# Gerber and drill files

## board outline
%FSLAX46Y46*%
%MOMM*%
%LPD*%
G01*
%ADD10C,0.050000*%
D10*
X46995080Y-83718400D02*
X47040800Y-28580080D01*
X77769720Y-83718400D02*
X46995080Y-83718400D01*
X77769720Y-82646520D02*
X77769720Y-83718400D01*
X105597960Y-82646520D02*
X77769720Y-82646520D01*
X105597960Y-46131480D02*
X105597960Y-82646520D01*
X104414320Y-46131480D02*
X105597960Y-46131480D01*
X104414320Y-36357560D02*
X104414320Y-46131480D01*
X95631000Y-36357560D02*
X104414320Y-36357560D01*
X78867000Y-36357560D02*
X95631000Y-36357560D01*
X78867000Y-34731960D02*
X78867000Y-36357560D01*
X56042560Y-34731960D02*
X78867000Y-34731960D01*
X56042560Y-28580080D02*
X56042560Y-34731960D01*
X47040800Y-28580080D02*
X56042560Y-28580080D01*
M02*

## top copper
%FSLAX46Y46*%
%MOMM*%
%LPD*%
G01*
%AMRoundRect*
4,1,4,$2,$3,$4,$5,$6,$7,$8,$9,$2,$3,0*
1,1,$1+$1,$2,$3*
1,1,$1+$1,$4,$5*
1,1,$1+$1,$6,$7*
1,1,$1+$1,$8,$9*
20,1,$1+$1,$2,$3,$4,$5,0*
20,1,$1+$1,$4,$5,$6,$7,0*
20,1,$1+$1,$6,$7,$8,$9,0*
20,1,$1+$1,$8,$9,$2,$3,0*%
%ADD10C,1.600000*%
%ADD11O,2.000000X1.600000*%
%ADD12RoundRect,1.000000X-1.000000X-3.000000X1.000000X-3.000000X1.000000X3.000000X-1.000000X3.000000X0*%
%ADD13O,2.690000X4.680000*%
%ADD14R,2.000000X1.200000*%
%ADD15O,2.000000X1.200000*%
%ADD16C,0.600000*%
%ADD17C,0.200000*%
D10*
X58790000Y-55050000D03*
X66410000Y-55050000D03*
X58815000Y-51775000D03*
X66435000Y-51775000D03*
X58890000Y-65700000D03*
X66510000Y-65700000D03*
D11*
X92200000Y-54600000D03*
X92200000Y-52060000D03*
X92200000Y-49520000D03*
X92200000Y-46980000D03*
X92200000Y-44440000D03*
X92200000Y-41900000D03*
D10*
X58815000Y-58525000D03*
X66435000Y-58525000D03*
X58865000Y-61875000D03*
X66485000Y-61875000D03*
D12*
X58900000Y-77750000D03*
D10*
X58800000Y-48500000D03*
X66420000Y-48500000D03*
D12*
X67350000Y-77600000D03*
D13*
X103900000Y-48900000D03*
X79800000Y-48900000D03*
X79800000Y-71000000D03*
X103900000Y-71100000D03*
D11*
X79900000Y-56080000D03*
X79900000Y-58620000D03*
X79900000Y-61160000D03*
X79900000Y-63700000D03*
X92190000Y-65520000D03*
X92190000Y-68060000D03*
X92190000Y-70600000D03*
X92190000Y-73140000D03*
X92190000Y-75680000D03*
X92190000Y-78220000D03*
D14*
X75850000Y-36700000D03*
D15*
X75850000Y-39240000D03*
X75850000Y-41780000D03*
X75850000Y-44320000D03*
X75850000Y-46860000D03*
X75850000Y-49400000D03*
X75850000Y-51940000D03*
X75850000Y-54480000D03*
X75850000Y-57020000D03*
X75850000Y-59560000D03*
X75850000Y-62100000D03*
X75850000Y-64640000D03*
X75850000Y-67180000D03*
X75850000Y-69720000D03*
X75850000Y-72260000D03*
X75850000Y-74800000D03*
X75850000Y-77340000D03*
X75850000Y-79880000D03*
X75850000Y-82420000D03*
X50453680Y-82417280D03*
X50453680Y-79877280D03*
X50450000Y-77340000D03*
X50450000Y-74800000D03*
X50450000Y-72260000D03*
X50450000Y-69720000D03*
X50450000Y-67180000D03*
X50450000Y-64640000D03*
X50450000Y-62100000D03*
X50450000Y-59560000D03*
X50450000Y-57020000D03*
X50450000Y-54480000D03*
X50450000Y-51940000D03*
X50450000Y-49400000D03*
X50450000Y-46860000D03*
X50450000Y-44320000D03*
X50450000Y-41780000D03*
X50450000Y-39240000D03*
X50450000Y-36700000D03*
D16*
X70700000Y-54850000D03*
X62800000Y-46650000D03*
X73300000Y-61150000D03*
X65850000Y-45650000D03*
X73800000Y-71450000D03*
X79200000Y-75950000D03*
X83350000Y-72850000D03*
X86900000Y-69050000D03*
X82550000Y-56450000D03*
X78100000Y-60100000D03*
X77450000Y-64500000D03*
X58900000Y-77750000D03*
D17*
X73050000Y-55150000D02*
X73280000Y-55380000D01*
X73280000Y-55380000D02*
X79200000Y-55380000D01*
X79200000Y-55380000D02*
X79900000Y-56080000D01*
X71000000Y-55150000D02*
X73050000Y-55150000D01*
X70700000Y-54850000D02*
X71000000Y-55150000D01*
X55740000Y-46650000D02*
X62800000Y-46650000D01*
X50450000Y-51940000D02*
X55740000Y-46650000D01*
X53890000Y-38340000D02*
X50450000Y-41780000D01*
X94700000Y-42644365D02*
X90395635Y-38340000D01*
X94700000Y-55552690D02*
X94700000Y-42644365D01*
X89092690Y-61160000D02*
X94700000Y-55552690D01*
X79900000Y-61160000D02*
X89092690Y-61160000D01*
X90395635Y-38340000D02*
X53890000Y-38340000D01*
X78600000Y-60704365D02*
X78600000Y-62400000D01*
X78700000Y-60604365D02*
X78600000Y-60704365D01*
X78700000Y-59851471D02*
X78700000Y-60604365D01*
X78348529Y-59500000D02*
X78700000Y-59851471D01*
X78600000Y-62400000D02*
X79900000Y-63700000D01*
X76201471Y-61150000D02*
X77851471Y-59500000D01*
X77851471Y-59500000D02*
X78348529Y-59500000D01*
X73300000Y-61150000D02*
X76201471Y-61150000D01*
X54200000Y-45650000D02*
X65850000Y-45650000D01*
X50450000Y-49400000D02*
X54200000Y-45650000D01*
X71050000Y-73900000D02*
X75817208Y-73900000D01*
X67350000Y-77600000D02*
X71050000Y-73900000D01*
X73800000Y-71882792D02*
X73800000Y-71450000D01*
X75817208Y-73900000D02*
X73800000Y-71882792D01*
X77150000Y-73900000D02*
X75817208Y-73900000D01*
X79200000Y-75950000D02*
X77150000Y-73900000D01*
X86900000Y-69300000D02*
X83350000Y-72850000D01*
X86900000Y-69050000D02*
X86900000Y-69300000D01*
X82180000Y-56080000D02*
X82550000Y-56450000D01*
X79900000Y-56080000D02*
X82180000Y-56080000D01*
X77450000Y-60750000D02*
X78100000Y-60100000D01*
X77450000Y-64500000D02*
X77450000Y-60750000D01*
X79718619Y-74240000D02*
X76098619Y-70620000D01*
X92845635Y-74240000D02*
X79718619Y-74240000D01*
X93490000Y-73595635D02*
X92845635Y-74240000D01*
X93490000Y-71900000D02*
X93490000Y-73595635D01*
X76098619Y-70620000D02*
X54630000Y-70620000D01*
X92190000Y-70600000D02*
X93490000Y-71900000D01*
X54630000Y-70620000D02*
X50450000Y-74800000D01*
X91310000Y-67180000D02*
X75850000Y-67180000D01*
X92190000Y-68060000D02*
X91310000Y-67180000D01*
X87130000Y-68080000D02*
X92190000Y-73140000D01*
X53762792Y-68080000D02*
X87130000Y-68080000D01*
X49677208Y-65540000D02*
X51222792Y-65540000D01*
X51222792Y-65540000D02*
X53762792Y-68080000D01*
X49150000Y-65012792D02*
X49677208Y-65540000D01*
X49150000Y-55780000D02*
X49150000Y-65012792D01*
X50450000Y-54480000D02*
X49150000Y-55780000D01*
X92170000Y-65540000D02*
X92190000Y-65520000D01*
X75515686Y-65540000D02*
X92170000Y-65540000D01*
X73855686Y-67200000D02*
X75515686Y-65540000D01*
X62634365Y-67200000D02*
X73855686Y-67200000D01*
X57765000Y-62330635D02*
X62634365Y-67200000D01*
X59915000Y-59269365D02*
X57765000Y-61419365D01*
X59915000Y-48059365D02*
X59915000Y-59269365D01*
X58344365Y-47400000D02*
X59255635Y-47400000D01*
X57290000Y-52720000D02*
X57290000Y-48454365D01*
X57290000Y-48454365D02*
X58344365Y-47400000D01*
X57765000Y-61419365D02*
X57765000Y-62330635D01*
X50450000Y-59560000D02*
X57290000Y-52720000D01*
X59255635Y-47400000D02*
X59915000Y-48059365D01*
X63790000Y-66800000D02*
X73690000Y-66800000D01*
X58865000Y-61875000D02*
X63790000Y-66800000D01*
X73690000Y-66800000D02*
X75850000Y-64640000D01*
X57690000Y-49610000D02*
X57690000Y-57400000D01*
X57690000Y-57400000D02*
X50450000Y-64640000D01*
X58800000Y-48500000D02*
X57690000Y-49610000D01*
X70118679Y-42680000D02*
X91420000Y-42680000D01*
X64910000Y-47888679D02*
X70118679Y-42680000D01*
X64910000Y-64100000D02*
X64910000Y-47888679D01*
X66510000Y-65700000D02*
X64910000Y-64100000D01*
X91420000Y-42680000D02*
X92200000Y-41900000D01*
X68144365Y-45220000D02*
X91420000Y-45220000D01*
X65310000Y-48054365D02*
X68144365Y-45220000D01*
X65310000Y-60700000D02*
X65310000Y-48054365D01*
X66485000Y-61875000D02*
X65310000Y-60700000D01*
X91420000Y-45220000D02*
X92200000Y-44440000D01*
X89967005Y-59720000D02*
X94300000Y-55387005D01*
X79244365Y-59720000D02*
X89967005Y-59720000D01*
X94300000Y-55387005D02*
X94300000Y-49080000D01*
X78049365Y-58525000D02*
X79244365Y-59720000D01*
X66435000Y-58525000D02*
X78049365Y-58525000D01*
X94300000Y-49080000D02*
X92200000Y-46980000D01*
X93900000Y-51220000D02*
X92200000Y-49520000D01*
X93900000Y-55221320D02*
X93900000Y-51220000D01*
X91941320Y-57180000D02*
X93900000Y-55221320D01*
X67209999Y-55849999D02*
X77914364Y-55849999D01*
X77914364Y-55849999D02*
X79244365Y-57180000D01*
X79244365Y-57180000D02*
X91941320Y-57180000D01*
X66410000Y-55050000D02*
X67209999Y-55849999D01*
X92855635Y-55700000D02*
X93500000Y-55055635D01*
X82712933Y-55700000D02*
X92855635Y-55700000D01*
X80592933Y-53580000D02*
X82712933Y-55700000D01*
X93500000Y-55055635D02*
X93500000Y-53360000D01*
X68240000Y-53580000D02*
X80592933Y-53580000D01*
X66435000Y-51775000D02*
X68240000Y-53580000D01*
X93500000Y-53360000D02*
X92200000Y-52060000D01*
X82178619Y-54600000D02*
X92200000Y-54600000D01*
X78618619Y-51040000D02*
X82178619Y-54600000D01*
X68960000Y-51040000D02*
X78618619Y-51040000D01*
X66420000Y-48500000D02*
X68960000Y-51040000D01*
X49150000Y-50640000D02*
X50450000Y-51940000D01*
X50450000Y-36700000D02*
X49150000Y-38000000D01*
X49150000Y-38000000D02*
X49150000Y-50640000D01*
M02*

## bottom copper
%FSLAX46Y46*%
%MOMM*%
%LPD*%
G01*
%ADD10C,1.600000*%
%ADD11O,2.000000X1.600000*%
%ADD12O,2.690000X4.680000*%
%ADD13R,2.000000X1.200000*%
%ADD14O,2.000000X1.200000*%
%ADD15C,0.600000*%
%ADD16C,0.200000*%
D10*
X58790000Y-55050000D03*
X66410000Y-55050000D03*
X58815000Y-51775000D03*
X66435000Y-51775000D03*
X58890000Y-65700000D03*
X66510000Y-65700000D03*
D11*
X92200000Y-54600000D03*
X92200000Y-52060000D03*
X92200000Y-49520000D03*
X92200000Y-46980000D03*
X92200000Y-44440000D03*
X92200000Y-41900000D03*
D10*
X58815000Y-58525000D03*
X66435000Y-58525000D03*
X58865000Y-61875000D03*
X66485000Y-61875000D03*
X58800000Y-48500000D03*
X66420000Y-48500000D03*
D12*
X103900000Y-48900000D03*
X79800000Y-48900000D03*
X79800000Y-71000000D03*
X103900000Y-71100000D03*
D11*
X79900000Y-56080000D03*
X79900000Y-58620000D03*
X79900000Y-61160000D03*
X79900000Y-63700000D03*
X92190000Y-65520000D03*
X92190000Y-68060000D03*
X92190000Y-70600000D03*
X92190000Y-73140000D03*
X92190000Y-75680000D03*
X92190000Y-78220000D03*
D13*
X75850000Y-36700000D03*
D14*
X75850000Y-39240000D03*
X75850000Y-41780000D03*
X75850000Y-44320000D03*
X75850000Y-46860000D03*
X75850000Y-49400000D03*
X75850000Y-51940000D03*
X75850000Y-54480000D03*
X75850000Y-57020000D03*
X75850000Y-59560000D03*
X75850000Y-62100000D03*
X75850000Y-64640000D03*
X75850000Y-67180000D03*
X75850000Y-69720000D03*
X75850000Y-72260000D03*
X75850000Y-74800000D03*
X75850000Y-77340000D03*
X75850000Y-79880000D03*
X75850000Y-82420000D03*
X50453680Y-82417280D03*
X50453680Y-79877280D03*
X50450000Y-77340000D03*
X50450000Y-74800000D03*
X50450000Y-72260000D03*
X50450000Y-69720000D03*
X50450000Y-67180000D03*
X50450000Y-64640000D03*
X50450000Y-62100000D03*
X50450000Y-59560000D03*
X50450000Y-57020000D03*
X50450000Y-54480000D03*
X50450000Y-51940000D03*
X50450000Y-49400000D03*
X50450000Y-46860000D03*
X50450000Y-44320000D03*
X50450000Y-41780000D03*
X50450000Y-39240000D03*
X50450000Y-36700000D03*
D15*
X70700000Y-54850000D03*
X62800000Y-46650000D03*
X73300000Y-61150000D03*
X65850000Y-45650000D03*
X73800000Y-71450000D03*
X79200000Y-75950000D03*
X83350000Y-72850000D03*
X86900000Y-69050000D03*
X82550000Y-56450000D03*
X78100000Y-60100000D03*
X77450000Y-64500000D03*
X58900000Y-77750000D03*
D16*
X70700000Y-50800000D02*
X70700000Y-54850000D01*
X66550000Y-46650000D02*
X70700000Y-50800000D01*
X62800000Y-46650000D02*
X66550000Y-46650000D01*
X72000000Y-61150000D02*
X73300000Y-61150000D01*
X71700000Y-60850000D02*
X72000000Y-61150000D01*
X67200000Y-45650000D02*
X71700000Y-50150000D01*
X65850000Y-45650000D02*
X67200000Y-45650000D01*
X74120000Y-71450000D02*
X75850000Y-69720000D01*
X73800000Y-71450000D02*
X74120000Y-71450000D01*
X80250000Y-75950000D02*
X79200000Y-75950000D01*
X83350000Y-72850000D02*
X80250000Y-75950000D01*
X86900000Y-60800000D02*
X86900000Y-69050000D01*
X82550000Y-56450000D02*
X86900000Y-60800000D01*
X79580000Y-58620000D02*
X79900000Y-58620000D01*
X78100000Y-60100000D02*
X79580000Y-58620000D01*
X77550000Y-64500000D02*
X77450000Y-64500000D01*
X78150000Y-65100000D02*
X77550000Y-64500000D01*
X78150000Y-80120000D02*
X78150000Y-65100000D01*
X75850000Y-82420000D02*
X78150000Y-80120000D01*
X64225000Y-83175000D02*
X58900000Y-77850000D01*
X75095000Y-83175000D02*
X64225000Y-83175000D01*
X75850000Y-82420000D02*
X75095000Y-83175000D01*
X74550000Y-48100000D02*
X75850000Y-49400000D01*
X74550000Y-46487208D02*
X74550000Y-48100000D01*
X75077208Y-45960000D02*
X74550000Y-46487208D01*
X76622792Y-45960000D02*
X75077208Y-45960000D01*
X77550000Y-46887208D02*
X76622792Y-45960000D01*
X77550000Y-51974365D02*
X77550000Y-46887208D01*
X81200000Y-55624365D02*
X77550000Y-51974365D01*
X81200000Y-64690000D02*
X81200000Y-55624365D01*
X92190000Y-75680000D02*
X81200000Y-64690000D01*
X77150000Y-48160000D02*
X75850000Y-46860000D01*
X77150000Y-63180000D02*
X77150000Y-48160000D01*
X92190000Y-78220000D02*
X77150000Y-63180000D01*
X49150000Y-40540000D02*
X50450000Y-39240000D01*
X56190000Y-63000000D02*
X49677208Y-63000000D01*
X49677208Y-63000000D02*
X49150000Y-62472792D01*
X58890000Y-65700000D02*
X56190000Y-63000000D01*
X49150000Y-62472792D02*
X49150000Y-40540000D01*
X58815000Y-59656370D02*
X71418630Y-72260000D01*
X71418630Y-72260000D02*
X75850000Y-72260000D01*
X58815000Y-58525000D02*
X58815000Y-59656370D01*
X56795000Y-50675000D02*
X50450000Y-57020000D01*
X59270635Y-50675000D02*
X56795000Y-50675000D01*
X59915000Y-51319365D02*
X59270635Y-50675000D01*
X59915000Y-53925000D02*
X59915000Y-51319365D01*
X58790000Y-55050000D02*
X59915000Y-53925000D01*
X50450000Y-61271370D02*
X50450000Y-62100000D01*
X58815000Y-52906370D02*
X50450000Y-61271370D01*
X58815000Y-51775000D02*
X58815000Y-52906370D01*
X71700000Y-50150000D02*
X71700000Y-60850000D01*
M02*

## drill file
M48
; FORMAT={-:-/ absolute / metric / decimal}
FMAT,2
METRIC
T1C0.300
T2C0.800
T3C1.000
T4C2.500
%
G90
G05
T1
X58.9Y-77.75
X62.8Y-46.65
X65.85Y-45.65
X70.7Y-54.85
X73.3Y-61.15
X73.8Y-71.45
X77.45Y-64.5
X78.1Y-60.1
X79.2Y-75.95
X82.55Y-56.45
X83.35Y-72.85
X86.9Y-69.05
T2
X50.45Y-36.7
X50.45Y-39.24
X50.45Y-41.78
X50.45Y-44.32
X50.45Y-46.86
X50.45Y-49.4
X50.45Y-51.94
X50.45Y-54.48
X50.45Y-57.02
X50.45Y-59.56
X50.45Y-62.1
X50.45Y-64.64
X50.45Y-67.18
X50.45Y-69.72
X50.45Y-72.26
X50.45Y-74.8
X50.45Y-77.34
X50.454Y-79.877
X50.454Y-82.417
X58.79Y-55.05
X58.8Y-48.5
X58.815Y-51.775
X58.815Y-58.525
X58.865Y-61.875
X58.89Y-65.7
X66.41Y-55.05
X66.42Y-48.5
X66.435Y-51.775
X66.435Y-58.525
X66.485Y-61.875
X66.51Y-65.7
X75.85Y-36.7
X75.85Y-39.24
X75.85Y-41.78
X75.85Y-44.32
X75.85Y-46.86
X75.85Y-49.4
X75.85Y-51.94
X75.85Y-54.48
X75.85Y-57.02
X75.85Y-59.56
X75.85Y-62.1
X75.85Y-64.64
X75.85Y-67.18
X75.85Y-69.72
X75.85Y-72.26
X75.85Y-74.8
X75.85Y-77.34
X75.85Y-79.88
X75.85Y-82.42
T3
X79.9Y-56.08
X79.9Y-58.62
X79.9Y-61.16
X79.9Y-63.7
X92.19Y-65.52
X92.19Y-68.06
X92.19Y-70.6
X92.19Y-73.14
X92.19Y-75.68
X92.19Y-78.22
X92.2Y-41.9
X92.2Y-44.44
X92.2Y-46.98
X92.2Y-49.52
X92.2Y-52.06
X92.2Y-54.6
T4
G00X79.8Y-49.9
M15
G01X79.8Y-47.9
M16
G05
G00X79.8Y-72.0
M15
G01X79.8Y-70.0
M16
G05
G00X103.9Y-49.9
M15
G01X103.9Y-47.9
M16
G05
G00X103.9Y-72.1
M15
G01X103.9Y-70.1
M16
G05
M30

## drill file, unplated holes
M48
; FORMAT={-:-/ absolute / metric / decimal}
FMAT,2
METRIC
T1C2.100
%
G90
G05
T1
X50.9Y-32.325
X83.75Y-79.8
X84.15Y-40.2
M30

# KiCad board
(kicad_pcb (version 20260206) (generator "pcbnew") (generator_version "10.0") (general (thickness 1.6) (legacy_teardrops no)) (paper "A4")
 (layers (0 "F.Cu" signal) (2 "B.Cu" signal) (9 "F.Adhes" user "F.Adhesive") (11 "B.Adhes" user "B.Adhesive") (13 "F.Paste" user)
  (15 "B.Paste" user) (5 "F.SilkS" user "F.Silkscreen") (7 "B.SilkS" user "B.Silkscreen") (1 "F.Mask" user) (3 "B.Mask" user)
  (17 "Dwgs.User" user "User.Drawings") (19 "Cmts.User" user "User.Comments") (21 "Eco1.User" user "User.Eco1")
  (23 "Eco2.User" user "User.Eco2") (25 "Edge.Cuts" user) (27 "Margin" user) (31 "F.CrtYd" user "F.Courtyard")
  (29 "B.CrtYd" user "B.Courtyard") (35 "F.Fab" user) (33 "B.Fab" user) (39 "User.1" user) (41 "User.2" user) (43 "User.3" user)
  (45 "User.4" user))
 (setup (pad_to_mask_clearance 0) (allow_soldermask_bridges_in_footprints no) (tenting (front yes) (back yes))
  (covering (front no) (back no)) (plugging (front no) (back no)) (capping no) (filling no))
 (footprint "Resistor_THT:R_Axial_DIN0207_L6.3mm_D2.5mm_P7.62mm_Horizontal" (layer "F.Cu") (at 58.79 55.05)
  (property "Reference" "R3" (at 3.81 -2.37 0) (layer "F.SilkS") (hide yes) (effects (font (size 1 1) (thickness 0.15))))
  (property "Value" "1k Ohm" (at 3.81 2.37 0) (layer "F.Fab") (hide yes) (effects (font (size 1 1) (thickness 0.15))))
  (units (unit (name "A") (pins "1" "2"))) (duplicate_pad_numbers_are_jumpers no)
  (pad "1" thru_hole circle (at 0 0) (size 1.6 1.6) (drill 0.8) (layers "*.Cu" "*.Mask") (remove_unused_layers no) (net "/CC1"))
  (pad "2" thru_hole circle (at 7.62 0) (size 1.6 1.6) (drill 0.8) (layers "*.Cu" "*.Mask") (remove_unused_layers no) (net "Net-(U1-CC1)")))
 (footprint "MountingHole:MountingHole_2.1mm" (layer "F.Cu") (at 50.9 32.325)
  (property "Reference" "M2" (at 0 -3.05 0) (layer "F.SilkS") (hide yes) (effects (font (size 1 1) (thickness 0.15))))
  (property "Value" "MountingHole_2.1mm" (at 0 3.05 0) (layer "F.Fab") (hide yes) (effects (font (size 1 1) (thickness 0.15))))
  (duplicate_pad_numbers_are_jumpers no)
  (pad "" np_thru_hole circle (at 0 0) (size 2.1 2.1) (drill 2.1) (layers "*.Cu" "*.Mask")))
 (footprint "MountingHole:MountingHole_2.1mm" (layer "F.Cu") (at 83.75 79.8)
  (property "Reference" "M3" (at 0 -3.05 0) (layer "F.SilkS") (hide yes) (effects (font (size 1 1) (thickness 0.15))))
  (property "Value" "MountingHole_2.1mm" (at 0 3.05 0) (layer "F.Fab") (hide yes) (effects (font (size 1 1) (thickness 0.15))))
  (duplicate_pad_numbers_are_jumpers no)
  (pad "" np_thru_hole circle (at 0 0) (size 2.1 2.1) (drill 2.1) (layers "*.Cu" "*.Mask")))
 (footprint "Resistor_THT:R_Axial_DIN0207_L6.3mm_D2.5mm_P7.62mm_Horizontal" (layer "F.Cu") (at 58.815 51.775)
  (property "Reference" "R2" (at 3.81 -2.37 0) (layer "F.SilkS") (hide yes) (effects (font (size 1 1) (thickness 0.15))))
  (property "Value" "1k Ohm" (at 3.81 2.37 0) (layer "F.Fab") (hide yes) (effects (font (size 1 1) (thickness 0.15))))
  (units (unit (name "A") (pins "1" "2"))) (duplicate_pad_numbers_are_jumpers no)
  (pad "1" thru_hole circle (at 0 0) (size 1.6 1.6) (drill 0.8) (layers "*.Cu" "*.Mask") (remove_unused_layers no) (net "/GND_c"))
  (pad "2" thru_hole circle (at 7.62 0) (size 1.6 1.6) (drill 0.8) (layers "*.Cu" "*.Mask") (remove_unused_layers no) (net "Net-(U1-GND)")))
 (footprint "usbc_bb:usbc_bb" (layer "F.Cu") (at 102.79 74.6 90)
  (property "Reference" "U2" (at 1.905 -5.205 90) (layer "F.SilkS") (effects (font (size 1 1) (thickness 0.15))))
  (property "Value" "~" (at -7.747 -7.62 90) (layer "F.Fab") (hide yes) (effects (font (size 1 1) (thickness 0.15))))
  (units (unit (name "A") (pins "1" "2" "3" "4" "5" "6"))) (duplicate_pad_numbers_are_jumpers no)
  (pad "1" thru_hole oval (at -3.62 -10.6 180) (size 2 1.6) (drill 1) (layers "*.Cu" "*.Mask") (remove_unused_layers no) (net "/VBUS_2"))
  (pad "2" thru_hole oval (at -1.08 -10.6 180) (size 2 1.6) (drill 1) (layers "*.Cu" "*.Mask") (remove_unused_layers no) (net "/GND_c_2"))
  (pad "3" thru_hole oval (at 1.46 -10.6 180) (size 2 1.6) (drill 1) (layers "*.Cu" "*.Mask") (remove_unused_layers no) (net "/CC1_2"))
  (pad "4" thru_hole oval (at 4 -10.6 180) (size 2 1.6) (drill 1) (layers "*.Cu" "*.Mask") (remove_unused_layers no) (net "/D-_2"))
  (pad "5" thru_hole oval (at 6.54 -10.6 180) (size 2 1.6) (drill 1) (layers "*.Cu" "*.Mask") (remove_unused_layers no) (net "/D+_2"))
  (pad "6" thru_hole oval (at 9.08 -10.6 180) (size 2 1.6) (drill 1) (layers "*.Cu" "*.Mask") (remove_unused_layers no) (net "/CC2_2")))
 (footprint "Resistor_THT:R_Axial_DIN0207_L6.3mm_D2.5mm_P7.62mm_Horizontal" (layer "F.Cu") (at 58.89 65.7)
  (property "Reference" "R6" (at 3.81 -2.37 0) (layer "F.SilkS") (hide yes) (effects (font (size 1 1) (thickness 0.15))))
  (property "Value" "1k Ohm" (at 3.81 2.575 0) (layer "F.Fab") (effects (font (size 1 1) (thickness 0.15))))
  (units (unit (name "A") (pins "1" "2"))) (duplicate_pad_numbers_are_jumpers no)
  (pad "1" thru_hole circle (at 0 0) (size 1.6 1.6) (drill 0.8) (layers "*.Cu" "*.Mask") (remove_unused_layers no) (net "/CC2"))
  (pad "2" thru_hole circle (at 7.62 0) (size 1.6 1.6) (drill 0.8) (layers "*.Cu" "*.Mask") (remove_unused_layers no) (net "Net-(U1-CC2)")))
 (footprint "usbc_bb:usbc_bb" (layer "F.Cu") (at 102.8 50.98 90)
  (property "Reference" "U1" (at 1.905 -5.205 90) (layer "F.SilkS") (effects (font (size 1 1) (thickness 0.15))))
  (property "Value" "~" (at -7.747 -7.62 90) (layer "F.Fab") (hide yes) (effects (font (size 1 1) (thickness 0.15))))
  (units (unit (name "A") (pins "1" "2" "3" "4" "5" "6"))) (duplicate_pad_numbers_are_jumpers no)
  (pad "1" thru_hole oval (at -3.62 -10.6 180) (size 2 1.6) (drill 1) (layers "*.Cu" "*.Mask") (remove_unused_layers no)
   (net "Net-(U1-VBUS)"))
  (pad "2" thru_hole oval (at -1.08 -10.6 180) (size 2 1.6) (drill 1) (layers "*.Cu" "*.Mask") (remove_unused_layers no)
   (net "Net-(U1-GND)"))
  (pad "3" thru_hole oval (at 1.46 -10.6 180) (size 2 1.6) (drill 1) (layers "*.Cu" "*.Mask") (remove_unused_layers no) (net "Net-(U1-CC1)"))
  (pad "4" thru_hole oval (at 4 -10.6 180) (size 2 1.6) (drill 1) (layers "*.Cu" "*.Mask") (remove_unused_layers no) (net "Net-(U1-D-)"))
  (pad "5" thru_hole oval (at 6.54 -10.6 180) (size 2 1.6) (drill 1) (layers "*.Cu" "*.Mask") (remove_unused_layers no) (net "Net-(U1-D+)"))
  (pad "6" thru_hole oval (at 9.08 -10.6 180) (size 2 1.6) (drill 1) (layers "*.Cu" "*.Mask") (remove_unused_layers no) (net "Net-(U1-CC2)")))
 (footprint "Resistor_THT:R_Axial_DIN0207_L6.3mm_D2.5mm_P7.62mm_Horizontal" (layer "F.Cu") (at 58.815 58.525)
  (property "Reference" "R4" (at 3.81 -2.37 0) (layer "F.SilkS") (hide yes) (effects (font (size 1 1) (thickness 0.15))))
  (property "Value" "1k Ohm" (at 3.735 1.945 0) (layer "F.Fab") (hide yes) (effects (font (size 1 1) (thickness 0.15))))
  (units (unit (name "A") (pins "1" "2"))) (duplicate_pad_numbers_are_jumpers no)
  (pad "1" thru_hole circle (at 0 0) (size 1.6 1.6) (drill 0.8) (layers "*.Cu" "*.Mask") (remove_unused_layers no) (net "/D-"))
  (pad "2" thru_hole circle (at 7.62 0) (size 1.6 1.6) (drill 0.8) (layers "*.Cu" "*.Mask") (remove_unused_layers no) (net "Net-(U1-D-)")))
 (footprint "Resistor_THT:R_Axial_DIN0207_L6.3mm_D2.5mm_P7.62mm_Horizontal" (layer "F.Cu") (at 58.865 61.875)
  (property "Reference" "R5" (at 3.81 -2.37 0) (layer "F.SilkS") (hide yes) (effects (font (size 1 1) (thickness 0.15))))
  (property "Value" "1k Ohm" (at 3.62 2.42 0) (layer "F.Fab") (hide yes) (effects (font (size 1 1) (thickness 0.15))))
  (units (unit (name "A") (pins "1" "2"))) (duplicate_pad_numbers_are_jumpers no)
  (pad "1" thru_hole circle (at 0 0) (size 1.6 1.6) (drill 0.8) (layers "*.Cu" "*.Mask") (remove_unused_layers no) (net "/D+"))
  (pad "2" thru_hole circle (at 7.62 0) (size 1.6 1.6) (drill 0.8) (layers "*.Cu" "*.Mask") (remove_unused_layers no) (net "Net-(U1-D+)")))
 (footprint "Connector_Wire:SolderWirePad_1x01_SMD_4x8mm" (layer "F.Cu") (at 58.9 77.75)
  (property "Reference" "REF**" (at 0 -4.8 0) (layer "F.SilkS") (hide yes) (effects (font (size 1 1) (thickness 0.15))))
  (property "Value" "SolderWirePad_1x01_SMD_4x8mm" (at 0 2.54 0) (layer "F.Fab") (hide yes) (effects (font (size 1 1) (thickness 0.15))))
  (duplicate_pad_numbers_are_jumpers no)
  (pad "1" smd roundrect (at 0 0) (size 4 8) (layers "F.Cu" "F.Mask") (roundrect_rratio 0.25) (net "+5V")))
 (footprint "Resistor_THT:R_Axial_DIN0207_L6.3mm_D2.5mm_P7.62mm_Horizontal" (layer "F.Cu") (at 58.8 48.5)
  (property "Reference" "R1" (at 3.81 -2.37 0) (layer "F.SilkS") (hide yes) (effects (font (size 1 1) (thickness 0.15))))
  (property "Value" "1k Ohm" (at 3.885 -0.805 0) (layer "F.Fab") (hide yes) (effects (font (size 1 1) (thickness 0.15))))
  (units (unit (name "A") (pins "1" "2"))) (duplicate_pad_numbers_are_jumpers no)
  (pad "1" thru_hole circle (at 0 0) (size 1.6 1.6) (drill 0.8) (layers "*.Cu" "*.Mask") (remove_unused_layers no) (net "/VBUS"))
  (pad "2" thru_hole circle (at 7.62 0) (size 1.6 1.6) (drill 0.8) (layers "*.Cu" "*.Mask") (remove_unused_layers no) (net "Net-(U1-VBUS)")))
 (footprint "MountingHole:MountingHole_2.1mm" (layer "F.Cu") (at 84.15 40.2)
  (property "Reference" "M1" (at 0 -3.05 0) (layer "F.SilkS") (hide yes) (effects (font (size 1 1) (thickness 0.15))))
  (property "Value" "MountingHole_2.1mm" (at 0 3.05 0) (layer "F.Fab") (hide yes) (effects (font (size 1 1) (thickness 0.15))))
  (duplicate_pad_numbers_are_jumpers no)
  (pad "" np_thru_hole circle (at 0 0) (size 2.1 2.1) (drill 2.1) (layers "*.Cu" "*.Mask")))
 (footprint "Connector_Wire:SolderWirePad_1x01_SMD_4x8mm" (layer "F.Cu") (at 67.35 77.6)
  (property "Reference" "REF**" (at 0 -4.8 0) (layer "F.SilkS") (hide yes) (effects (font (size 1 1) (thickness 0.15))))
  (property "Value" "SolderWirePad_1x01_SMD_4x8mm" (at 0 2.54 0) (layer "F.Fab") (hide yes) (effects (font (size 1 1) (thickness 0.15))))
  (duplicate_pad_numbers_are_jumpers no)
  (pad "1" smd roundrect (at 0 0) (size 4 8) (layers "F.Cu" "F.Mask") (roundrect_rratio 0.25) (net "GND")))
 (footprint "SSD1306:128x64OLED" (layer "B.Cu") (at 90.5 59.7 -90)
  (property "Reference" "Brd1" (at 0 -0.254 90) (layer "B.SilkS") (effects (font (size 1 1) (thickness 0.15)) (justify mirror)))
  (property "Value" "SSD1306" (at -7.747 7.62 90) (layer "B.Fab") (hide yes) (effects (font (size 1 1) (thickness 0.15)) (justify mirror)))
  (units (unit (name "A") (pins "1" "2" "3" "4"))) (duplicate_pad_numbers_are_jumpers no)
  (pad "" thru_hole oval (at -10.8 -13.4 90) (size 4.68 2.69) (drill oval 4.5 2.5) (layers "*.Cu" "*.Mask") (remove_unused_layers no))
  (pad "" thru_hole oval (at -10.8 10.7 90) (size 4.68 2.69) (drill oval 4.5 2.5) (layers "*.Cu" "*.Mask") (remove_unused_layers no))
  (pad "" thru_hole oval (at 11.3 10.7 90) (size 4.68 2.69) (drill oval 4.5 2.5) (layers "*.Cu" "*.Mask") (remove_unused_layers no))
  (pad "" thru_hole oval (at 11.4 -13.4 90) (size 4.68 2.69) (drill oval 4.5 2.5) (layers "*.Cu" "*.Mask") (remove_unused_layers no))
  (pad "1" thru_hole oval (at -3.62 10.6 180) (size 2 1.6) (drill 1) (layers "*.Cu" "*.Mask") (remove_unused_layers no) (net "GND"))
  (pad "2" thru_hole oval (at -1.08 10.6 180) (size 2 1.6) (drill 1) (layers "*.Cu" "*.Mask") (remove_unused_layers no) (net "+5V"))
  (pad "3" thru_hole oval (at 1.46 10.6 180) (size 2 1.6) (drill 1) (layers "*.Cu" "*.Mask") (remove_unused_layers no) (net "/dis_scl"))
  (pad "4" thru_hole oval (at 4 10.6 180) (size 2 1.6) (drill 1) (layers "*.Cu" "*.Mask") (remove_unused_layers no) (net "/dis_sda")))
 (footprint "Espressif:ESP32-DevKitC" (layer "B.Cu") (at 75.85 36.7 180)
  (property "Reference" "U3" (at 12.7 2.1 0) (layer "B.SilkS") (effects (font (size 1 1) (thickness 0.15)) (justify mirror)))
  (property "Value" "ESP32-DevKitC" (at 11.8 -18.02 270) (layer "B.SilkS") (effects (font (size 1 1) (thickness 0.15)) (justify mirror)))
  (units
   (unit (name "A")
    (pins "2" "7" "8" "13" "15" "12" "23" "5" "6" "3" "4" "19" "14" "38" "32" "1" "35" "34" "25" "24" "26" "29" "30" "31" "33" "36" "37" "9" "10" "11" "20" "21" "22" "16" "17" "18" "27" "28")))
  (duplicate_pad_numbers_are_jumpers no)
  (pad "1" thru_hole rect (at 0 0 270) (size 1.2 2) (drill 0.8) (layers "*.Cu" "*.Mask") (remove_unused_layers no) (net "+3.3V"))
  (pad "2" thru_hole oval (at 0 -2.54 270) (size 1.2 2) (drill 0.8) (layers "*.Cu" "*.Mask") (remove_unused_layers no)
   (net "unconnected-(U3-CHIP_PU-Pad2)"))
  (pad "3" thru_hole oval (at 0 -5.08 270) (size 1.2 2) (drill 0.8) (layers "*.Cu" "*.Mask") (remove_unused_layers no)
   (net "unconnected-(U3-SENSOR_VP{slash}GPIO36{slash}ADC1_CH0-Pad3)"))
  (pad "4" thru_hole oval (at 0 -7.62 270) (size 1.2 2) (drill 0.8) (layers "*.Cu" "*.Mask") (remove_unused_layers no)
   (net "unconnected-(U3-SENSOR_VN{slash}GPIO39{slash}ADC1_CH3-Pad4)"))
  (pad "5" thru_hole oval (at 0 -10.16 270) (size 1.2 2) (drill 0.8) (layers "*.Cu" "*.Mask") (remove_unused_layers no) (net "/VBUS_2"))
  (pad "6" thru_hole oval (at 0 -12.7 270) (size 1.2 2) (drill 0.8) (layers "*.Cu" "*.Mask") (remove_unused_layers no) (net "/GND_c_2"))
  (pad "7" thru_hole oval (at 0 -15.24 270) (size 1.2 2) (drill 0.8) (layers "*.Cu" "*.Mask") (remove_unused_layers no)
   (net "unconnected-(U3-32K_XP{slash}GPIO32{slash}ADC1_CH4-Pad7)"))
  (pad "8" thru_hole oval (at 0 -17.78 270) (size 1.2 2) (drill 0.8) (layers "*.Cu" "*.Mask") (remove_unused_layers no)
   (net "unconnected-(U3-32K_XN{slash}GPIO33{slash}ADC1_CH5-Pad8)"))
  (pad "9" thru_hole oval (at 0 -20.32 270) (size 1.2 2) (drill 0.8) (layers "*.Cu" "*.Mask") (remove_unused_layers no)
   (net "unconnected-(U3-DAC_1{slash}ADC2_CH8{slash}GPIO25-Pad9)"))
  (pad "10" thru_hole oval (at 0 -22.86 270) (size 1.2 2) (drill 0.8) (layers "*.Cu" "*.Mask") (remove_unused_layers no)
   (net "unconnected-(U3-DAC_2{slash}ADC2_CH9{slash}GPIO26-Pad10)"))
  (pad "11" thru_hole oval (at 0 -25.4 270) (size 1.2 2) (drill 0.8) (layers "*.Cu" "*.Mask") (remove_unused_layers no)
   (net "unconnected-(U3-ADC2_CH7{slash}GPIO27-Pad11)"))
  (pad "12" thru_hole oval (at 0 -27.94 270) (size 1.2 2) (drill 0.8) (layers "*.Cu" "*.Mask") (remove_unused_layers no) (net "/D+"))
  (pad "13" thru_hole oval (at 0 -30.48 270) (size 1.2 2) (drill 0.8) (layers "*.Cu" "*.Mask") (remove_unused_layers no) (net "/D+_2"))
  (pad "14" thru_hole oval (at 0 -33.02 270) (size 1.2 2) (drill 0.8) (layers "*.Cu" "*.Mask") (remove_unused_layers no) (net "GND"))
  (pad "15" thru_hole oval (at 0 -35.56 270) (size 1.2 2) (drill 0.8) (layers "*.Cu" "*.Mask") (remove_unused_layers no) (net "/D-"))
  (pad "16" thru_hole oval (at 0 -38.1 270) (size 1.2 2) (drill 0.8) (layers "*.Cu" "*.Mask") (remove_unused_layers no)
   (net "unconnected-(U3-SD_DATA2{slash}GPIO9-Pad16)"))
  (pad "17" thru_hole oval (at 0 -40.64 270) (size 1.2 2) (drill 0.8) (layers "*.Cu" "*.Mask") (remove_unused_layers no)
   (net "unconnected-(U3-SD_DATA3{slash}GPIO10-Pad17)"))
  (pad "18" thru_hole oval (at 0 -43.18 270) (size 1.2 2) (drill 0.8) (layers "*.Cu" "*.Mask") (remove_unused_layers no)
   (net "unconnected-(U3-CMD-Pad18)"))
  (pad "19" thru_hole oval (at 0 -45.72 270) (size 1.2 2) (drill 0.8) (layers "*.Cu" "*.Mask") (remove_unused_layers no) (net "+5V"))
  (pad "20" thru_hole oval (at 25.39632 -45.71728 270) (size 1.2 2) (drill 0.8) (layers "*.Cu" "*.Mask") (remove_unused_layers no)
   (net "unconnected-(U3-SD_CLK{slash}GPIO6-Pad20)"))
  (pad "21" thru_hole oval (at 25.39632 -43.17728 270) (size 1.2 2) (drill 0.8) (layers "*.Cu" "*.Mask") (remove_unused_layers no)
   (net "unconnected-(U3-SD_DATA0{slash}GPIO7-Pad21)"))
  (pad "22" thru_hole oval (at 25.4 -40.64 270) (size 1.2 2) (drill 0.8) (layers "*.Cu" "*.Mask") (remove_unused_layers no)
   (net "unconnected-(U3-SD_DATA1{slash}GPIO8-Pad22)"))
  (pad "23" thru_hole oval (at 25.4 -38.1 270) (size 1.2 2) (drill 0.8) (layers "*.Cu" "*.Mask") (remove_unused_layers no) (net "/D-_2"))
  (pad "24" thru_hole oval (at 25.4 -35.56 270) (size 1.2 2) (drill 0.8) (layers "*.Cu" "*.Mask") (remove_unused_layers no)
   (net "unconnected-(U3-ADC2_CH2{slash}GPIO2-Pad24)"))
  (pad "25" thru_hole oval (at 25.4 -33.02 270) (size 1.2 2) (drill 0.8) (layers "*.Cu" "*.Mask") (remove_unused_layers no)
   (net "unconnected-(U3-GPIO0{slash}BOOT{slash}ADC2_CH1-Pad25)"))
  (pad "26" thru_hole oval (at 25.4 -30.48 270) (size 1.2 2) (drill 0.8) (layers "*.Cu" "*.Mask") (remove_unused_layers no)
   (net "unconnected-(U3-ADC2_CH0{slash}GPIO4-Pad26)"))
  (pad "27" thru_hole oval (at 25.4 -27.94 270) (size 1.2 2) (drill 0.8) (layers "*.Cu" "*.Mask") (remove_unused_layers no) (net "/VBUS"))
  (pad "28" thru_hole oval (at 25.4 -25.4 270) (size 1.2 2) (drill 0.8) (layers "*.Cu" "*.Mask") (remove_unused_layers no) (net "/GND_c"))
  (pad "29" thru_hole oval (at 25.4 -22.86 270) (size 1.2 2) (drill 0.8) (layers "*.Cu" "*.Mask") (remove_unused_layers no) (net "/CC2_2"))
  (pad "30" thru_hole oval (at 25.4 -20.32 270) (size 1.2 2) (drill 0.8) (layers "*.Cu" "*.Mask") (remove_unused_layers no) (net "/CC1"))
  (pad "31" thru_hole oval (at 25.4 -17.78 270) (size 1.2 2) (drill 0.8) (layers "*.Cu" "*.Mask") (remove_unused_layers no) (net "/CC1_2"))
  (pad "32" thru_hole oval (at 25.4 -15.24 270) (size 1.2 2) (drill 0.8) (layers "*.Cu" "*.Mask") (remove_unused_layers no) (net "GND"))
  (pad "33" thru_hole oval (at 25.4 -12.7 270) (size 1.2 2) (drill 0.8) (layers "*.Cu" "*.Mask") (remove_unused_layers no) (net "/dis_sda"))
  (pad "34" thru_hole oval (at 25.4 -10.16 270) (size 1.2 2) (drill 0.8) (layers "*.Cu" "*.Mask") (remove_unused_layers no)
   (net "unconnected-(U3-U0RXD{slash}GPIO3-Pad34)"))
  (pad "35" thru_hole oval (at 25.4 -7.62 270) (size 1.2 2) (drill 0.8) (layers "*.Cu" "*.Mask") (remove_unused_layers no)
   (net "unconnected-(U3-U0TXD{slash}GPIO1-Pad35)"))
  (pad "36" thru_hole oval (at 25.4 -5.08 270) (size 1.2 2) (drill 0.8) (layers "*.Cu" "*.Mask") (remove_unused_layers no) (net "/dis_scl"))
  (pad "37" thru_hole oval (at 25.4 -2.54 270) (size 1.2 2) (drill 0.8) (layers "*.Cu" "*.Mask") (remove_unused_layers no) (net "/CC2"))
  (pad "38" thru_hole oval (at 25.4 0 270) (size 1.2 2) (drill 0.8) (layers "*.Cu" "*.Mask") (remove_unused_layers no) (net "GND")))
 (gr_line (start 46.99508 83.7184) (end 47.0408 28.58008) (stroke (width 0.05) (type default)) (layer "Edge.Cuts"))
 (gr_line (start 47.0408 28.58008) (end 56.04256 28.58008) (stroke (width 0.05) (type default)) (layer "Edge.Cuts"))
 (gr_line (start 56.04256 28.58008) (end 56.04256 34.73196) (stroke (width 0.05) (type default)) (layer "Edge.Cuts"))
 (gr_line (start 56.04256 34.73196) (end 78.867 34.73196) (stroke (width 0.05) (type default)) (layer "Edge.Cuts"))
 (gr_line (start 77.76972 82.64652) (end 77.76972 83.7184) (stroke (width 0.05) (type default)) (layer "Edge.Cuts"))
 (gr_line (start 77.76972 83.7184) (end 46.99508 83.7184) (stroke (width 0.05) (type default)) (layer "Edge.Cuts"))
 (gr_line (start 78.867 34.73196) (end 78.867 36.35756) (stroke (width 0.05) (type default)) (layer "Edge.Cuts"))
 (gr_line (start 78.867 36.35756) (end 95.631 36.35756) (stroke (width 0.05) (type default)) (layer "Edge.Cuts"))
 (gr_line (start 95.631 36.35756) (end 104.41432 36.35756) (stroke (width 0.05) (type default)) (layer "Edge.Cuts"))
 (gr_line (start 104.41432 36.35756) (end 104.41432 46.13148) (stroke (width 0.05) (type default)) (layer "Edge.Cuts"))
 (gr_line (start 104.41432 46.13148) (end 105.59796 46.13148) (stroke (width 0.05) (type default)) (layer "Edge.Cuts"))
 (gr_line (start 105.59796 46.13148) (end 105.59796 82.64652) (stroke (width 0.05) (type default)) (layer "Edge.Cuts"))
 (gr_line (start 105.59796 82.64652) (end 77.76972 82.64652) (stroke (width 0.05) (type default)) (layer "Edge.Cuts"))
 (segment (start 58.79 55.05) (end 59.915 53.925) (width 0.2) (layer "B.Cu") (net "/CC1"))
 (segment (start 59.270635 50.675) (end 56.795 50.675) (width 0.2) (layer "B.Cu") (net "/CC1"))
 (segment (start 59.915 51.319365) (end 59.270635 50.675) (width 0.2) (layer "B.Cu") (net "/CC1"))
 (segment (start 56.795 50.675) (end 50.45 57.02) (width 0.2) (layer "B.Cu") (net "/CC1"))
 (segment (start 59.915 53.925) (end 59.915 51.319365) (width 0.2) (layer "B.Cu") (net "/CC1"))
 (segment (start 79.244365 57.18) (end 91.94132 57.18) (width 0.2) (layer "F.Cu") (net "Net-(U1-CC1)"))
 (segment (start 67.209999 55.849999) (end 77.914364 55.849999) (width 0.2) (layer "F.Cu") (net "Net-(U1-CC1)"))
 (segment (start 77.914364 55.849999) (end 79.244365 57.18) (width 0.2) (layer "F.Cu") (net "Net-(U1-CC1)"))
 (segment (start 93.9 51.22) (end 92.2 49.52) (width 0.2) (layer "F.Cu") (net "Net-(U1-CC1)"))
 (segment (start 66.41 55.05) (end 67.209999 55.849999) (width 0.2) (layer "F.Cu") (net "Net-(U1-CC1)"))
 (segment (start 91.94132 57.18) (end 93.9 55.22132) (width 0.2) (layer "F.Cu") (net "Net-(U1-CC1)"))
 (segment (start 93.9 55.22132) (end 93.9 51.22) (width 0.2) (layer "F.Cu") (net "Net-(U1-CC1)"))
 (segment (start 50.45 61.27137) (end 50.45 62.1) (width 0.2) (layer "B.Cu") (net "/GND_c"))
 (segment (start 58.815 51.775) (end 58.815 52.90637) (width 0.2) (layer "B.Cu") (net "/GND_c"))
 (segment (start 58.815 52.90637) (end 50.45 61.27137) (width 0.2) (layer "B.Cu") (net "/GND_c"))
 (segment (start 80.592933 53.58) (end 82.712933 55.7) (width 0.2) (layer "F.Cu") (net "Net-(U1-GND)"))
 (segment (start 82.712933 55.7) (end 92.855635 55.7) (width 0.2) (layer "F.Cu") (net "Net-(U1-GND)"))
 (segment (start 66.435 51.775) (end 68.24 53.58) (width 0.2) (layer "F.Cu") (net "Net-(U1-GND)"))
 (segment (start 92.855635 55.7) (end 93.5 55.055635) (width 0.2) (layer "F.Cu") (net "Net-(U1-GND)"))
 (segment (start 93.5 55.055635) (end 93.5 53.36) (width 0.2) (layer "F.Cu") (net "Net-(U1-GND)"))
 (segment (start 93.5 53.36) (end 92.2 52.06) (width 0.2) (layer "F.Cu") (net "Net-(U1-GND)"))
 (segment (start 68.24 53.58) (end 80.592933 53.58) (width 0.2) (layer "F.Cu") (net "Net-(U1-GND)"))
 (segment (start 92.19 78.22) (end 77.15 63.18) (width 0.2) (layer "B.Cu") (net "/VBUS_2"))
 (segment (start 77.15 63.18) (end 77.15 48.16) (width 0.2) (layer "B.Cu") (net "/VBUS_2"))
 (segment (start 77.15 48.16) (end 75.85 46.86) (width 0.2) (layer "B.Cu") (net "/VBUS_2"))
 (segment (start 75.077208 45.96) (end 74.55 46.487208) (width 0.2) (layer "B.Cu") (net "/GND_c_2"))
 (segment (start 81.2 64.69) (end 81.2 55.624365) (width 0.2) (layer "B.Cu") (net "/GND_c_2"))
 (segment (start 81.2 55.624365) (end 77.55 51.974365) (width 0.2) (layer "B.Cu") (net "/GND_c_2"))
 (segment (start 74.55 48.1) (end 75.85 49.4) (width 0.2) (layer "B.Cu") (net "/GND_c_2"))
 (segment (start 74.55 46.487208) (end 74.55 48.1) (width 0.2) (layer "B.Cu") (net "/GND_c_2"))
 (segment (start 76.622792 45.96) (end 75.077208 45.96) (width 0.2) (layer "B.Cu") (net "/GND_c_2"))
 (segment (start 92.19 75.68) (end 81.2 64.69) (width 0.2) (layer "B.Cu") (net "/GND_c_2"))
 (segment (start 77.55 51.974365) (end 77.55 46.887208) (width 0.2) (layer "B.Cu") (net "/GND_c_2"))
 (segment (start 77.55 46.887208) (end 76.622792 45.96) (width 0.2) (layer "B.Cu") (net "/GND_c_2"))
 (segment (start 49.15 65.012792) (end 49.677208 65.54) (width 0.2) (layer "F.Cu") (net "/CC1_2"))
 (segment (start 51.222792 65.54) (end 53.762792 68.08) (width 0.2) (layer "F.Cu") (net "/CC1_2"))
 (segment (start 49.677208 65.54) (end 51.222792 65.54) (width 0.2) (layer "F.Cu") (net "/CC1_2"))
 (segment (start 50.45 54.48) (end 49.15 55.78) (width 0.2) (layer "F.Cu") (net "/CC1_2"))
 (segment (start 49.15 55.78) (end 49.15 65.012792) (width 0.2) (layer "F.Cu") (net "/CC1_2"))
 (segment (start 53.762792 68.08) (end 87.13 68.08) (width 0.2) (layer "F.Cu") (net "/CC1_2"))
 (segment (start 87.13 68.08) (end 92.19 73.14) (width 0.2) (layer "F.Cu") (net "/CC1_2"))
 (segment (start 92.19 70.6) (end 93.49 71.9) (width 0.2) (layer "F.Cu") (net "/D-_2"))
 (segment (start 93.49 73.595635) (end 92.845635 74.24) (width 0.2) (layer "F.Cu") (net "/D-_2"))
 (segment (start 93.49 71.9) (end 93.49 73.595635) (width 0.2) (layer "F.Cu") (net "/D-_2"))
 (segment (start 79.718619 74.24) (end 76.098619 70.62) (width 0.2) (layer "F.Cu") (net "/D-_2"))
 (segment (start 54.63 70.62) (end 50.45 74.8) (width 0.2) (layer "F.Cu") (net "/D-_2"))
 (segment (start 76.098619 70.62) (end 54.63 70.62) (width 0.2) (layer "F.Cu") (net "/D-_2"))
 (segment (start 92.845635 74.24) (end 79.718619 74.24) (width 0.2) (layer "F.Cu") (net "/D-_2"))
 (segment (start 91.31 67.18) (end 75.85 67.18) (width 0.2) (layer "F.Cu") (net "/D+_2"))
 (segment (start 92.19 68.06) (end 91.31 67.18) (width 0.2) (layer "F.Cu") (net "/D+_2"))
 (segment (start 92.17 65.54) (end 92.19 65.52) (width 0.2) (layer "F.Cu") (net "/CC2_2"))
 (segment (start 75.515686 65.54) (end 92.17 65.54) (width 0.2) (layer "F.Cu") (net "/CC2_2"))
 (segment (start 73.855686 67.2) (end 75.515686 65.54) (width 0.2) (layer "F.Cu") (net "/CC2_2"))
 (segment (start 58.344365 47.4) (end 59.255635 47.4) (width 0.2) (layer "F.Cu") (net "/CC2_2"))
 (segment (start 59.255635 47.4) (end 59.915 48.059365) (width 0.2) (layer "F.Cu") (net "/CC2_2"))
 (segment (start 57.765 61.419365) (end 57.765 62.330635) (width 0.2) (layer "F.Cu") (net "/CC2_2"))
 (segment (start 59.915 59.269365) (end 57.765 61.419365) (width 0.2) (layer "F.Cu") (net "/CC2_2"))
 (segment (start 57.765 62.330635) (end 62.634365 67.2) (width 0.2) (layer "F.Cu") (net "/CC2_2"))
 (segment (start 59.915 48.059365) (end 59.915 59.269365) (width 0.2) (layer "F.Cu") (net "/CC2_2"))
 (segment (start 62.634365 67.2) (end 73.855686 67.2) (width 0.2) (layer "F.Cu") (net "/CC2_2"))
 (segment (start 57.29 48.454365) (end 58.344365 47.4) (width 0.2) (layer "F.Cu") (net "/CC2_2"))
 (segment (start 57.29 52.72) (end 57.29 48.454365) (width 0.2) (layer "F.Cu") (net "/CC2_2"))
 (segment (start 50.45 59.56) (end 57.29 52.72) (width 0.2) (layer "F.Cu") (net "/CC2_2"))
 (segment (start 49.15 62.472792) (end 49.15 40.54) (width 0.2) (layer "B.Cu") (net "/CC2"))
 (segment (start 49.15 40.54) (end 50.45 39.24) (width 0.2) (layer "B.Cu") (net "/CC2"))
 (segment (start 58.89 65.7) (end 56.19 63) (width 0.2) (layer "B.Cu") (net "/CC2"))
 (segment (start 56.19 63) (end 49.677208 63) (width 0.2) (layer "B.Cu") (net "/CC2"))
 (segment (start 49.677208 63) (end 49.15 62.472792) (width 0.2) (layer "B.Cu") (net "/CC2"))
 (segment (start 64.91 47.888679) (end 70.118679 42.68) (width 0.2) (layer "F.Cu") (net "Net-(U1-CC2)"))
 (segment (start 91.42 42.68) (end 92.2 41.9) (width 0.2) (layer "F.Cu") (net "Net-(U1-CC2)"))
 (segment (start 70.118679 42.68) (end 91.42 42.68) (width 0.2) (layer "F.Cu") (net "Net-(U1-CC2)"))
 (segment (start 66.51 65.7) (end 64.91 64.1) (width 0.2) (layer "F.Cu") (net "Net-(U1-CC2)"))
 (segment (start 64.91 64.1) (end 64.91 47.888679) (width 0.2) (layer "F.Cu") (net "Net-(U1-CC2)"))
 (segment (start 66.42 48.5) (end 68.96 51.04) (width 0.2) (layer "F.Cu") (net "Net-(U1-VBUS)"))
 (segment (start 68.96 51.04) (end 78.618619 51.04) (width 0.2) (layer "F.Cu") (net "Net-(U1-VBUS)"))
 (segment (start 82.178619 54.6) (end 92.2 54.6) (width 0.2) (layer "F.Cu") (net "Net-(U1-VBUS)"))
 (segment (start 78.618619 51.04) (end 82.178619 54.6) (width 0.2) (layer "F.Cu") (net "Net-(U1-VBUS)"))
 (segment (start 79.244365 59.72) (end 89.967005 59.72) (width 0.2) (layer "F.Cu") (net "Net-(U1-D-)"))
 (segment (start 94.3 55.387005) (end 94.3 49.08) (width 0.2) (layer "F.Cu") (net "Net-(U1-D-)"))
 (segment (start 66.435 58.525) (end 78.049365 58.525) (width 0.2) (layer "F.Cu") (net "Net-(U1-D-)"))
 (segment (start 89.967005 59.72) (end 94.3 55.387005) (width 0.2) (layer "F.Cu") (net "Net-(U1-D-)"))
 (segment (start 78.049365 58.525) (end 79.244365 59.72) (width 0.2) (layer "F.Cu") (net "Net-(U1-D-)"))
 (segment (start 94.3 49.08) (end 92.2 46.98) (width 0.2) (layer "F.Cu") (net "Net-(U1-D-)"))
 (segment (start 65.31 48.054365) (end 68.144365 45.22) (width 0.2) (layer "F.Cu") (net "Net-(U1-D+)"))
 (segment (start 68.144365 45.22) (end 91.42 45.22) (width 0.2) (layer "F.Cu") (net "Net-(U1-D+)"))
 (segment (start 65.31 60.7) (end 65.31 48.054365) (width 0.2) (layer "F.Cu") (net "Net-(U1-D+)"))
 (segment (start 91.42 45.22) (end 92.2 44.44) (width 0.2) (layer "F.Cu") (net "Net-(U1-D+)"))
 (segment (start 66.485 61.875) (end 65.31 60.7) (width 0.2) (layer "F.Cu") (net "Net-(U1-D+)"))
 (segment (start 58.815 58.525) (end 58.815 59.65637) (width 0.2) (layer "B.Cu") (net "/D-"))
 (segment (start 58.815 59.65637) (end 71.41863 72.26) (width 0.2) (layer "B.Cu") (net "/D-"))
 (segment (start 71.41863 72.26) (end 75.85 72.26) (width 0.2) (layer "B.Cu") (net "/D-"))
 (segment (start 73.69 66.8) (end 75.85 64.64) (width 0.2) (layer "F.Cu") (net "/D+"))
 (segment (start 63.79 66.8) (end 73.69 66.8) (width 0.2) (layer "F.Cu") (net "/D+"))
 (segment (start 58.865 61.875) (end 63.79 66.8) (width 0.2) (layer "F.Cu") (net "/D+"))
 (segment (start 77.45 64.5) (end 77.45 60.75) (width 0.2) (layer "F.Cu") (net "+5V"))
 (segment (start 77.45 60.75) (end 78.1 60.1) (width 0.2) (layer "F.Cu") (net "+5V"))
 (via (at 77.45 64.5) (size 0.6) (drill 0.3) (layers "F.Cu" "B.Cu") (free yes) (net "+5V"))
 (via (at 78.1 60.1) (size 0.6) (drill 0.3) (layers "F.Cu" "B.Cu") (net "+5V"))
 (via (at 58.9 77.75) (size 0.6) (drill 0.3) (layers "F.Cu" "B.Cu") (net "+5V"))
 (segment (start 75.85 82.42) (end 75.095 83.175) (width 0.2) (layer "B.Cu") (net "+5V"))
 (segment (start 75.095 83.175) (end 64.225 83.175) (width 0.2) (layer "B.Cu") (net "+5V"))
 (segment (start 77.55 64.5) (end 77.45 64.5) (width 0.2) (layer "B.Cu") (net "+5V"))
 (segment (start 75.85 82.42) (end 78.15 80.12) (width 0.2) (layer "B.Cu") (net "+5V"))
 (segment (start 64.225 83.175) (end 58.9 77.85) (width 0.2) (layer "B.Cu") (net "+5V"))
 (segment (start 79.58 58.62) (end 79.9 58.62) (width 0.2) (layer "B.Cu") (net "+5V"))
 (segment (start 78.15 65.1) (end 77.55 64.5) (width 0.2) (layer "B.Cu") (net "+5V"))
 (segment (start 78.1 60.1) (end 79.58 58.62) (width 0.2) (layer "B.Cu") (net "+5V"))
 (segment (start 78.15 80.12) (end 78.15 65.1) (width 0.2) (layer "B.Cu") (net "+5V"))
 (segment (start 57.69 57.4) (end 50.45 64.64) (width 0.2) (layer "F.Cu") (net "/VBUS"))
 (segment (start 57.69 49.61) (end 57.69 57.4) (width 0.2) (layer "F.Cu") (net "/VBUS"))
 (segment (start 58.8 48.5) (end 57.69 49.61) (width 0.2) (layer "F.Cu") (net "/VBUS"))
 (segment (start 71.05 73.9) (end 75.817208 73.9) (width 0.2) (layer "F.Cu") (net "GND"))
 (segment (start 50.45 51.94) (end 55.74 46.65) (width 0.2) (layer "F.Cu") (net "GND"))
 (segment (start 73.05 55.15) (end 73.28 55.38) (width 0.2) (layer "F.Cu") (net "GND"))
 (segment (start 79.2 75.95) (end 77.15 73.9) (width 0.2) (layer "F.Cu") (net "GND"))
 (segment (start 75.817208 73.9) (end 73.8 71.882792) (width 0.2) (layer "F.Cu") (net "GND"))
 (segment (start 49.15 38) (end 49.15 50.64) (width 0.2) (layer "F.Cu") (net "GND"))
 (segment (start 77.15 73.9) (end 75.817208 73.9) (width 0.2) (layer "F.Cu") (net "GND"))
 (segment (start 50.45 36.7) (end 49.15 38) (width 0.2) (layer "F.Cu") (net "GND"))
 (segment (start 49.15 50.64) (end 50.45 51.94) (width 0.2) (layer "F.Cu") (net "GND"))
 (segment (start 86.9 69.05) (end 86.9 69.3) (width 0.2) (layer "F.Cu") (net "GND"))
 (segment (start 79.2 55.38) (end 79.9 56.08) (width 0.2) (layer "F.Cu") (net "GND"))
 (segment (start 73.8 71.882792) (end 73.8 71.45) (width 0.2) (layer "F.Cu") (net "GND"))
 (segment (start 55.74 46.65) (end 62.8 46.65) (width 0.2) (layer "F.Cu") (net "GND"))
 (segment (start 82.18 56.08) (end 82.55 56.45) (width 0.2) (layer "F.Cu") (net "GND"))
 (segment (start 86.9 69.3) (end 83.35 72.85) (width 0.2) (layer "F.Cu") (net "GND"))
 (segment (start 73.28 55.38) (end 79.2 55.38) (width 0.2) (layer "F.Cu") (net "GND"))
 (segment (start 70.7 54.85) (end 71 55.15) (width 0.2) (layer "F.Cu") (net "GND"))
 (segment (start 71 55.15) (end 73.05 55.15) (width 0.2) (layer "F.Cu") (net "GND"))
 (segment (start 67.35 77.6) (end 71.05 73.9) (width 0.2) (layer "F.Cu") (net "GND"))
 (segment (start 79.9 56.08) (end 82.18 56.08) (width 0.2) (layer "F.Cu") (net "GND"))
 (via (at 79.2 75.95) (size 0.6) (drill 0.3) (layers "F.Cu" "B.Cu") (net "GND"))
 (via (at 73.8 71.45) (size 0.6) (drill 0.3) (layers "F.Cu" "B.Cu") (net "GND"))
 (via (at 70.7 54.85) (size 0.6) (drill 0.3) (layers "F.Cu" "B.Cu") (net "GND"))
 (via (at 62.8 46.65) (size 0.6) (drill 0.3) (layers "F.Cu" "B.Cu") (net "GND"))
 (via (at 86.9 69.05) (size 0.6) (drill 0.3) (layers "F.Cu" "B.Cu") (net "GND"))
 (via (at 82.55 56.45) (size 0.6) (drill 0.3) (layers "F.Cu" "B.Cu") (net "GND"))
 (via (at 83.35 72.85) (size 0.6) (drill 0.3) (layers "F.Cu" "B.Cu") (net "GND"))
 (segment (start 74.12 71.45) (end 75.85 69.72) (width 0.2) (layer "B.Cu") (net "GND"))
 (segment (start 80.25 75.95) (end 79.2 75.95) (width 0.2) (layer "B.Cu") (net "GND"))
 (segment (start 66.55 46.65) (end 70.7 50.8) (width 0.2) (layer "B.Cu") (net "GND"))
 (segment (start 70.7 50.8) (end 70.7 54.85) (width 0.2) (layer "B.Cu") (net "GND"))
 (segment (start 83.35 72.85) (end 80.25 75.95) (width 0.2) (layer "B.Cu") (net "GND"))
 (segment (start 82.55 56.45) (end 86.9 60.8) (width 0.2) (layer "B.Cu") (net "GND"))
 (segment (start 73.8 71.45) (end 74.12 71.45) (width 0.2) (layer "B.Cu") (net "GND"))
 (segment (start 86.9 60.8) (end 86.9 69.05) (width 0.2) (layer "B.Cu") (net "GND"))
 (segment (start 62.8 46.65) (end 66.55 46.65) (width 0.2) (layer "B.Cu") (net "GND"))
 (segment (start 79.9 61.16) (end 89.09269 61.16) (width 0.2) (layer "F.Cu") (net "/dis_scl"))
 (segment (start 94.7 42.644365) (end 90.395635 38.34) (width 0.2) (layer "F.Cu") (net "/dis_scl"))
 (segment (start 90.395635 38.34) (end 53.89 38.34) (width 0.2) (layer "F.Cu") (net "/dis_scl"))
 (segment (start 94.7 55.55269) (end 94.7 42.644365) (width 0.2) (layer "F.Cu") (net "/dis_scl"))
 (segment (start 53.89 38.34) (end 50.45 41.78) (width 0.2) (layer "F.Cu") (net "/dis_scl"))
 (segment (start 89.09269 61.16) (end 94.7 55.55269) (width 0.2) (layer "F.Cu") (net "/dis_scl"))
 (segment (start 78.7 60.604365) (end 78.6 60.704365) (width 0.2) (layer "F.Cu") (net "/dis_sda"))
 (segment (start 54.2 45.65) (end 65.85 45.65) (width 0.2) (layer "F.Cu") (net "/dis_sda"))
 (segment (start 78.348529 59.5) (end 78.7 59.851471) (width 0.2) (layer "F.Cu") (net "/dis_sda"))
 (segment (start 50.45 49.4) (end 54.2 45.65) (width 0.2) (layer "F.Cu") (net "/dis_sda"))
 (segment (start 76.201471 61.15) (end 77.851471 59.5) (width 0.2) (layer "F.Cu") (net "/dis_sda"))
 (segment (start 78.6 62.4) (end 79.9 63.7) (width 0.2) (layer "F.Cu") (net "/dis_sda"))
 (segment (start 78.6 60.704365) (end 78.6 62.4) (width 0.2) (layer "F.Cu") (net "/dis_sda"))
 (segment (start 78.7 59.851471) (end 78.7 60.604365) (width 0.2) (layer "F.Cu") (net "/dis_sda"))
 (segment (start 73.3 61.15) (end 76.201471 61.15) (width 0.2) (layer "F.Cu") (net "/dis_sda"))
 (segment (start 77.851471 59.5) (end 78.348529 59.5) (width 0.2) (layer "F.Cu") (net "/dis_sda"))
 (via (at 65.85 45.65) (size 0.6) (drill 0.3) (layers "F.Cu" "B.Cu") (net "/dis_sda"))
 (via (at 73.3 61.15) (size 0.6) (drill 0.3) (layers "F.Cu" "B.Cu") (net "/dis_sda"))
 (segment (start 71.7 50.15) (end 71.7 60.85) (width 0.2) (layer "B.Cu") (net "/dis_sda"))
 (segment (start 67.2 45.65) (end 71.7 50.15) (width 0.2) (layer "B.Cu") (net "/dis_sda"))
 (segment (start 71.7 60.85) (end 72 61.15) (width 0.2) (layer "B.Cu") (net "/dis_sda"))
 (segment (start 72 61.15) (end 73.3 61.15) (width 0.2) (layer "B.Cu") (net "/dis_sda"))
 (segment (start 65.85 45.65) (end 67.2 45.65) (width 0.2) (layer "B.Cu") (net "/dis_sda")))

